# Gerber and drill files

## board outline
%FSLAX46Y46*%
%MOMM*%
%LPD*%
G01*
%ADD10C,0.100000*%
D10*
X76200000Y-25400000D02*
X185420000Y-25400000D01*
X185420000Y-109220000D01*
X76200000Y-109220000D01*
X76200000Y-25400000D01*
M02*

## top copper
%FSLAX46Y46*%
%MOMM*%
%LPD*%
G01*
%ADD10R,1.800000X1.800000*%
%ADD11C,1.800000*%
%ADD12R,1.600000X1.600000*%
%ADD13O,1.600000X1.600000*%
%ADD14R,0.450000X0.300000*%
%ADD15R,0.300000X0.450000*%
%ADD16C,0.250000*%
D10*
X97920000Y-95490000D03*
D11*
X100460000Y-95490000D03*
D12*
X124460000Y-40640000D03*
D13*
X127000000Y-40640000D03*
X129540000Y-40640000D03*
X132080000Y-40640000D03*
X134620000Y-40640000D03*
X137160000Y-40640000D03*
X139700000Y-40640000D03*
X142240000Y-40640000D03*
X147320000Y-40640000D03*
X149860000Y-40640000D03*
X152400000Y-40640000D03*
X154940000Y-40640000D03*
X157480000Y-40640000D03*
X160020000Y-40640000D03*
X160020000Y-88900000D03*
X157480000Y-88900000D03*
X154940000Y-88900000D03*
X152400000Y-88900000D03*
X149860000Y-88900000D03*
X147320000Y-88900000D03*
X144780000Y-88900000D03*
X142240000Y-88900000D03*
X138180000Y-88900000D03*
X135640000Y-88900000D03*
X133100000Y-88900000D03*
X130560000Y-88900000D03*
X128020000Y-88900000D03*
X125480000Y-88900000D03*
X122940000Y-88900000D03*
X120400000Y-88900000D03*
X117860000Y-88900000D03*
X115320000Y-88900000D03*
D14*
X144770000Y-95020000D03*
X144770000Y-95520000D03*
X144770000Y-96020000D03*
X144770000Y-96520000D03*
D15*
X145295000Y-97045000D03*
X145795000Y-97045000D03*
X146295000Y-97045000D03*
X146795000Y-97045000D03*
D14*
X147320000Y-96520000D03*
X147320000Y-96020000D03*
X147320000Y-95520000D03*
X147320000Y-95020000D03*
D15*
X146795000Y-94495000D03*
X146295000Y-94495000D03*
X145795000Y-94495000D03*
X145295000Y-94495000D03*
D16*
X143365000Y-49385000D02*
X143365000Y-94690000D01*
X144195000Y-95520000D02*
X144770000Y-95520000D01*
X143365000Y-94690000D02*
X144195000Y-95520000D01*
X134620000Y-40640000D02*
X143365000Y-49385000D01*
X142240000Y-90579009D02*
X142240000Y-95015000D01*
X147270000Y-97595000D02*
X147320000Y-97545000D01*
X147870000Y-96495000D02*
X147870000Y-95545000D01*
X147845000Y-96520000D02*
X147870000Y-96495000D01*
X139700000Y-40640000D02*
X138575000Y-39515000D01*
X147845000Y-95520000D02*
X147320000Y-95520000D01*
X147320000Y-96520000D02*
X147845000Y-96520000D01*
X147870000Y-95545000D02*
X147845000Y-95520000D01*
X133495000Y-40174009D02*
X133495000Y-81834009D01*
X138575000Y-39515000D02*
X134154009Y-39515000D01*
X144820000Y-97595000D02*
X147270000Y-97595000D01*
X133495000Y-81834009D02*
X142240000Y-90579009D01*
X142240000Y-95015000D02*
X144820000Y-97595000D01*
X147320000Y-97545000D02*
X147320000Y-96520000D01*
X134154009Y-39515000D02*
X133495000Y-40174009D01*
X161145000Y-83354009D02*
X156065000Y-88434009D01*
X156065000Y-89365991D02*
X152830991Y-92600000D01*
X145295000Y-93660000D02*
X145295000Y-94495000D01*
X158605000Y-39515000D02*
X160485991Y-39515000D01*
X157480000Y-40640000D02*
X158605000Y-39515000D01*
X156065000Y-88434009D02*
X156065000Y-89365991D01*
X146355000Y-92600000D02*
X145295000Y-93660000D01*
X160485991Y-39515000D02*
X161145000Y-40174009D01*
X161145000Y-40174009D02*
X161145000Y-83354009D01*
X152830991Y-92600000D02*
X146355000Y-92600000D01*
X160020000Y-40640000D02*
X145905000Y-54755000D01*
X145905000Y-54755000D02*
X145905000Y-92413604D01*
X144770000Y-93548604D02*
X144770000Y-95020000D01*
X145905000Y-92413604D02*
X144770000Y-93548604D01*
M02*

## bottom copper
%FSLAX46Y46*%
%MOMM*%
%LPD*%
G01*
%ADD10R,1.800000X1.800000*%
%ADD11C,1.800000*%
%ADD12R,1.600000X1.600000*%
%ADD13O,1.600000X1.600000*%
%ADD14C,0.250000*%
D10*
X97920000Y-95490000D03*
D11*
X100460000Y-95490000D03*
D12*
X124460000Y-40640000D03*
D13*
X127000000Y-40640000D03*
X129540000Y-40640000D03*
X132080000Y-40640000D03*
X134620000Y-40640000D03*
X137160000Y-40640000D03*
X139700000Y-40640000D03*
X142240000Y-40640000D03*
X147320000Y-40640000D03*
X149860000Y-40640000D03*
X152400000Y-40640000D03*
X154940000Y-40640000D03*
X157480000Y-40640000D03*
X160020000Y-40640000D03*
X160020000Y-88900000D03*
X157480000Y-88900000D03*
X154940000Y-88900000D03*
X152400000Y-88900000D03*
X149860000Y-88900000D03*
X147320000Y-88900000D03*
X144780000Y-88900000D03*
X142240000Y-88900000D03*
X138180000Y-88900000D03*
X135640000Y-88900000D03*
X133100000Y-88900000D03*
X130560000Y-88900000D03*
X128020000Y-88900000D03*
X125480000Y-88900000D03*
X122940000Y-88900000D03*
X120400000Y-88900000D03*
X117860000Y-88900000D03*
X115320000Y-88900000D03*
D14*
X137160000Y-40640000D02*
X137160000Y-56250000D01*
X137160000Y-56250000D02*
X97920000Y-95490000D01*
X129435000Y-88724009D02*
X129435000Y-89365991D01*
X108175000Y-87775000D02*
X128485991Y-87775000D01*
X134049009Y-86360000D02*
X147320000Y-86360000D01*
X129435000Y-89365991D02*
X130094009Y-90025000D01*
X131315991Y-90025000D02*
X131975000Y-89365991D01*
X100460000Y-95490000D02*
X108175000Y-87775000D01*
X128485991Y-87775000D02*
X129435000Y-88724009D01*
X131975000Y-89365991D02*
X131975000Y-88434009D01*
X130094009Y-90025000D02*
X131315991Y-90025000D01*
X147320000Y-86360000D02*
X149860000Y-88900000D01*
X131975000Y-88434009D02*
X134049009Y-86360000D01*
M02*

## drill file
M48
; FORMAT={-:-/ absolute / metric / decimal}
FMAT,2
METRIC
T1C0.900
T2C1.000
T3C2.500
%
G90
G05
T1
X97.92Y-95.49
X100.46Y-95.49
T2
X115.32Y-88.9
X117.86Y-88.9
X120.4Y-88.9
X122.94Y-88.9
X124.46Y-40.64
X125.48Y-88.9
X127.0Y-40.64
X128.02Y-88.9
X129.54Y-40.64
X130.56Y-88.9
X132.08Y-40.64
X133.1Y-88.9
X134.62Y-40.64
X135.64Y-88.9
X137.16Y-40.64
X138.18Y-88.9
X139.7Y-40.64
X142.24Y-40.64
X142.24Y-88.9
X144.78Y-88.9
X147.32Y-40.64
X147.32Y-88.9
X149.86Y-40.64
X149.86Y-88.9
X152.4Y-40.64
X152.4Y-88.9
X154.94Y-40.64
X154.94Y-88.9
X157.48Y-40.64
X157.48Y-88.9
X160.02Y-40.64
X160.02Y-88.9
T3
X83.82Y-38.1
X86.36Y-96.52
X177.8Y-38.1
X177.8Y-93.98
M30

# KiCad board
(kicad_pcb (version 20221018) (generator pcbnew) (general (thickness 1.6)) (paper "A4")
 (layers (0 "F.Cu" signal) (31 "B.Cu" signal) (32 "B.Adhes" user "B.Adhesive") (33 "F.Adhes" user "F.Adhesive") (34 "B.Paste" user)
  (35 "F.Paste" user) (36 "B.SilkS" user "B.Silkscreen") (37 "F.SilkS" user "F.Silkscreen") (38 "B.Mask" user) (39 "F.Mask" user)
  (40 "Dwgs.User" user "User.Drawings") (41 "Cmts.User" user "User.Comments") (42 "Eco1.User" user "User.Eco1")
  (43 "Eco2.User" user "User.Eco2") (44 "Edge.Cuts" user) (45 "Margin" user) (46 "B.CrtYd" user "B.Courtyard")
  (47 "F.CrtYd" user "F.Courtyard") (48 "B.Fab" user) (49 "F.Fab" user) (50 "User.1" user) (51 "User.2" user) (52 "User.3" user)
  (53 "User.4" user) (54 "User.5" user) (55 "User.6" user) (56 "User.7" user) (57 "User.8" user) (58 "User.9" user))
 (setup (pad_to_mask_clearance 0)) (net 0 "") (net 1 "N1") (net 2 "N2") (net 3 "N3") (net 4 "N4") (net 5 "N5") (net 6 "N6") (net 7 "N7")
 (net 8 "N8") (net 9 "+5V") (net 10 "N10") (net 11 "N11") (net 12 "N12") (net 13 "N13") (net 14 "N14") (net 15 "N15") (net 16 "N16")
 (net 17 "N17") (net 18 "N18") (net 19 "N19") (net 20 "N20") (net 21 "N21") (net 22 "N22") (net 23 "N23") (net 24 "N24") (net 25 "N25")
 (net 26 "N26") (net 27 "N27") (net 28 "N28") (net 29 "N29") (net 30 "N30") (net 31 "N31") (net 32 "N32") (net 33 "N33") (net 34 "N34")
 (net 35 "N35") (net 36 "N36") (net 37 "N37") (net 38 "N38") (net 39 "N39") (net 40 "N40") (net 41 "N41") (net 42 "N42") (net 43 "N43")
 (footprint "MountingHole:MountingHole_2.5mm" (layer "F.Cu") (at 83.82 38.1)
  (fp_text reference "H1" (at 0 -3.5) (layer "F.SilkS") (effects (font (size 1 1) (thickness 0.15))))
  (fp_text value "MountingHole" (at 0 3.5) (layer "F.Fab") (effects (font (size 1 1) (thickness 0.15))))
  (pad "" np_thru_hole circle (at 0 0) (size 2.5 2.5) (drill 2.5) (layers "*.Cu" "*.Mask")))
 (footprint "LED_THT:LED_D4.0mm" (layer "F.Cu") (at 97.92 95.49)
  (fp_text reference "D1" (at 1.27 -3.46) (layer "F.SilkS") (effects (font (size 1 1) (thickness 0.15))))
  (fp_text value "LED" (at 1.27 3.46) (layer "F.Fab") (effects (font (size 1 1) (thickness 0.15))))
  (pad "1" thru_hole rect (at 0 0) (size 1.8 1.8) (drill 0.9) (layers "*.Cu" "*.Mask") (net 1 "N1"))
  (pad "2" thru_hole circle (at 2.54 0) (size 1.8 1.8) (drill 0.9) (layers "*.Cu" "*.Mask") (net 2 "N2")))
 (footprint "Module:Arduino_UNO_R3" (layer "F.Cu") (at 124.46 40.64)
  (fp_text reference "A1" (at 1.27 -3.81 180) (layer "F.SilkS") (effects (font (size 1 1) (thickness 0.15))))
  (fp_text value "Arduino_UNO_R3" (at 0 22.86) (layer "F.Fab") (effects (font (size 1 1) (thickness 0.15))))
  (pad "1" thru_hole rect (at 0 0 90) (size 1.6 1.6) (drill 1) (layers "*.Cu" "*.Mask") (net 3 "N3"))
  (pad "2" thru_hole oval (at 2.54 0 90) (size 1.6 1.6) (drill 1) (layers "*.Cu" "*.Mask") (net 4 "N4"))
  (pad "3" thru_hole oval (at 5.08 0 90) (size 1.6 1.6) (drill 1) (layers "*.Cu" "*.Mask") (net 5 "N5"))
  (pad "4" thru_hole oval (at 7.62 0 90) (size 1.6 1.6) (drill 1) (layers "*.Cu" "*.Mask") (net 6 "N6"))
  (pad "5" thru_hole oval (at 10.16 0 90) (size 1.6 1.6) (drill 1) (layers "*.Cu" "*.Mask") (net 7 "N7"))
  (pad "6" thru_hole oval (at 12.7 0 90) (size 1.6 1.6) (drill 1) (layers "*.Cu" "*.Mask") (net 1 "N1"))
  (pad "7" thru_hole oval (at 15.24 0 90) (size 1.6 1.6) (drill 1) (layers "*.Cu" "*.Mask") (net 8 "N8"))
  (pad "8" thru_hole oval (at 17.78 0 90) (size 1.6 1.6) (drill 1) (layers "*.Cu" "*.Mask") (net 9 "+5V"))
  (pad "9" thru_hole oval (at 22.86 0 90) (size 1.6 1.6) (drill 1) (layers "*.Cu" "*.Mask") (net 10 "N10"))
  (pad "10" thru_hole oval (at 25.4 0 90) (size 1.6 1.6) (drill 1) (layers "*.Cu" "*.Mask") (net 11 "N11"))
  (pad "11" thru_hole oval (at 27.94 0 90) (size 1.6 1.6) (drill 1) (layers "*.Cu" "*.Mask") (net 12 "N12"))
  (pad "12" thru_hole oval (at 30.48 0 90) (size 1.6 1.6) (drill 1) (layers "*.Cu" "*.Mask") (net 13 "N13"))
  (pad "13" thru_hole oval (at 33.02 0 90) (size 1.6 1.6) (drill 1) (layers "*.Cu" "*.Mask") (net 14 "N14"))
  (pad "14" thru_hole oval (at 35.56 0 90) (size 1.6 1.6) (drill 1) (layers "*.Cu" "*.Mask") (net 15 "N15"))
  (pad "15" thru_hole oval (at 35.56 48.26 90) (size 1.6 1.6) (drill 1) (layers "*.Cu" "*.Mask") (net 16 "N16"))
  (pad "16" thru_hole oval (at 33.02 48.26 90) (size 1.6 1.6) (drill 1) (layers "*.Cu" "*.Mask") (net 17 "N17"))
  (pad "17" thru_hole oval (at 30.48 48.26 90) (size 1.6 1.6) (drill 1) (layers "*.Cu" "*.Mask") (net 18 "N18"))
  (pad "18" thru_hole oval (at 27.94 48.26 90) (size 1.6 1.6) (drill 1) (layers "*.Cu" "*.Mask") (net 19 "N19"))
  (pad "19" thru_hole oval (at 25.4 48.26 90) (size 1.6 1.6) (drill 1) (layers "*.Cu" "*.Mask") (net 2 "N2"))
  (pad "20" thru_hole oval (at 22.86 48.26 90) (size 1.6 1.6) (drill 1) (layers "*.Cu" "*.Mask") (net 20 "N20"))
  (pad "21" thru_hole oval (at 20.32 48.26 90) (size 1.6 1.6) (drill 1) (layers "*.Cu" "*.Mask") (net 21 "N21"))
  (pad "22" thru_hole oval (at 17.78 48.26 90) (size 1.6 1.6) (drill 1) (layers "*.Cu" "*.Mask") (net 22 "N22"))
  (pad "23" thru_hole oval (at 13.72 48.26 90) (size 1.6 1.6) (drill 1) (layers "*.Cu" "*.Mask") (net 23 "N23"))
  (pad "24" thru_hole oval (at 11.18 48.26 90) (size 1.6 1.6) (drill 1) (layers "*.Cu" "*.Mask") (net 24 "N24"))
  (pad "25" thru_hole oval (at 8.64 48.26 90) (size 1.6 1.6) (drill 1) (layers "*.Cu" "*.Mask") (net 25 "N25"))
  (pad "26" thru_hole oval (at 6.1 48.26 90) (size 1.6 1.6) (drill 1) (layers "*.Cu" "*.Mask") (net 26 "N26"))
  (pad "27" thru_hole oval (at 3.56 48.26 90) (size 1.6 1.6) (drill 1) (layers "*.Cu" "*.Mask") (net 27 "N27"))
  (pad "28" thru_hole oval (at 1.02 48.26 90) (size 1.6 1.6) (drill 1) (layers "*.Cu" "*.Mask") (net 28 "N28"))
  (pad "29" thru_hole oval (at -1.52 48.26 90) (size 1.6 1.6) (drill 1) (layers "*.Cu" "*.Mask") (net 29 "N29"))
  (pad "30" thru_hole oval (at -4.06 48.26 90) (size 1.6 1.6) (drill 1) (layers "*.Cu" "*.Mask") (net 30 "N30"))
  (pad "31" thru_hole oval (at -6.6 48.26 90) (size 1.6 1.6) (drill 1) (layers "*.Cu" "*.Mask") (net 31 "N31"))
  (pad "32" thru_hole oval (at -9.14 48.26 90) (size 1.6 1.6) (drill 1) (layers "*.Cu" "*.Mask") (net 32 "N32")))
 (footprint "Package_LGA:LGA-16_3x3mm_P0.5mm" (layer "F.Cu") (at 146.045 95.77)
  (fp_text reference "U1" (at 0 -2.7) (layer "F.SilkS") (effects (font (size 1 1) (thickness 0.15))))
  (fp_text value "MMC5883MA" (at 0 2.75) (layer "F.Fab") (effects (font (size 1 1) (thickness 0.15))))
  (pad "1" smd rect (at -1.275 -0.75 90) (size 0.3 0.45) (layers "F.Cu" "F.Paste" "F.Mask") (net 15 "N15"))
  (pad "2" smd rect (at -1.275 -0.25 90) (size 0.3 0.45) (layers "F.Cu" "F.Paste" "F.Mask") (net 7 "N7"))
  (pad "3" smd rect (at -1.275 0.25 90) (size 0.3 0.45) (layers "F.Cu" "F.Paste" "F.Mask") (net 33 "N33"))
  (pad "4" smd rect (at -1.275 0.75 90) (size 0.3 0.45) (layers "F.Cu" "F.Paste" "F.Mask") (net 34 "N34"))
  (pad "5" smd rect (at -0.75 1.275) (size 0.3 0.45) (layers "F.Cu" "F.Paste" "F.Mask") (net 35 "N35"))
  (pad "6" smd rect (at -0.25 1.275) (size 0.3 0.45) (layers "F.Cu" "F.Paste" "F.Mask") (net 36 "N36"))
  (pad "7" smd rect (at 0.25 1.275) (size 0.3 0.45) (layers "F.Cu" "F.Paste" "F.Mask") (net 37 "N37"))
  (pad "8" smd rect (at 0.75 1.275) (size 0.3 0.45) (layers "F.Cu" "F.Paste" "F.Mask") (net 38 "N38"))
  (pad "9" smd rect (at 1.275 0.75 90) (size 0.3 0.45) (layers "F.Cu" "F.Paste" "F.Mask") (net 8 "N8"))
  (pad "10" smd rect (at 1.275 0.25 90) (size 0.3 0.45) (layers "F.Cu" "F.Paste" "F.Mask") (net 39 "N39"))
  (pad "11" smd rect (at 1.275 -0.25 90) (size 0.3 0.45) (layers "F.Cu" "F.Paste" "F.Mask") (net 8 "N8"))
  (pad "12" smd rect (at 1.275 -0.75 90) (size 0.3 0.45) (layers "F.Cu" "F.Paste" "F.Mask") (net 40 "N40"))
  (pad "13" smd rect (at 0.75 -1.275) (size 0.3 0.45) (layers "F.Cu" "F.Paste" "F.Mask") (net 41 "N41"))
  (pad "14" smd rect (at 0.25 -1.275) (size 0.3 0.45) (layers "F.Cu" "F.Paste" "F.Mask") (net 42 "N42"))
  (pad "15" smd rect (at -0.25 -1.275) (size 0.3 0.45) (layers "F.Cu" "F.Paste" "F.Mask") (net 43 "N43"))
  (pad "16" smd rect (at -0.75 -1.275) (size 0.3 0.45) (layers "F.Cu" "F.Paste" "F.Mask") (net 14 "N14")))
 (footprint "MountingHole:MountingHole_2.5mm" (layer "F.Cu") (at 86.36 96.52)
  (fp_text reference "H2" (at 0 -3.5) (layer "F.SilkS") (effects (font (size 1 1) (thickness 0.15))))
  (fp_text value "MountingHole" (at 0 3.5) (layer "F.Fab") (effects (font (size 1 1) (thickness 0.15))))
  (pad "" np_thru_hole circle (at 0 0) (size 2.5 2.5) (drill 2.5) (layers "*.Cu" "*.Mask")))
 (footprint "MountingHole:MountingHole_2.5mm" (layer "F.Cu") (at 177.8 38.1)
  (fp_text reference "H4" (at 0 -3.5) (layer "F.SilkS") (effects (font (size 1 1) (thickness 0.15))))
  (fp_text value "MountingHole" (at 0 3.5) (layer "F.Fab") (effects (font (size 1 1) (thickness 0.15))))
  (pad "" np_thru_hole circle (at 0 0) (size 2.5 2.5) (drill 2.5) (layers "*.Cu" "*.Mask")))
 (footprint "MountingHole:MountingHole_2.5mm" (layer "F.Cu") (at 177.8 93.98)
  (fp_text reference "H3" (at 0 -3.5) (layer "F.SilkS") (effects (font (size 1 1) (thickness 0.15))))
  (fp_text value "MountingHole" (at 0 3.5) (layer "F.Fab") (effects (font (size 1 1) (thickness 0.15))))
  (pad "" np_thru_hole circle (at 0 0) (size 2.5 2.5) (drill 2.5) (layers "*.Cu" "*.Mask")))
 (gr_rect (start 76.2 25.4) (end 185.42 109.22) (stroke (width 0.1) (type default)) (fill none) (layer "Edge.Cuts"))
 (segment (start 143.365 49.385) (end 143.365 94.69) (width 0.25) (layer "F.Cu") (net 7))
 (segment (start 144.195 95.52) (end 144.77 95.52) (width 0.25) (layer "F.Cu") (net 7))
 (segment (start 143.365 94.69) (end 144.195 95.52) (width 0.25) (layer "F.Cu") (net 7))
 (segment (start 134.62 40.64) (end 143.365 49.385) (width 0.25) (layer "F.Cu") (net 7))
 (segment (start 137.16 40.64) (end 137.16 56.25) (width 0.25) (layer "B.Cu") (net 1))
 (segment (start 137.16 56.25) (end 97.92 95.49) (width 0.25) (layer "B.Cu") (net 1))
 (segment (start 142.24 90.579009) (end 142.24 95.015) (width 0.25) (layer "F.Cu") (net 8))
 (segment (start 147.27 97.595) (end 147.32 97.545) (width 0.25) (layer "F.Cu") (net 8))
 (segment (start 147.87 96.495) (end 147.87 95.545) (width 0.25) (layer "F.Cu") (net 8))
 (segment (start 147.845 96.52) (end 147.87 96.495) (width 0.25) (layer "F.Cu") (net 8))
 (segment (start 139.7 40.64) (end 138.575 39.515) (width 0.25) (layer "F.Cu") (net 8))
 (segment (start 147.845 95.52) (end 147.32 95.52) (width 0.25) (layer "F.Cu") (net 8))
 (segment (start 147.32 96.52) (end 147.845 96.52) (width 0.25) (layer "F.Cu") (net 8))
 (segment (start 147.87 95.545) (end 147.845 95.52) (width 0.25) (layer "F.Cu") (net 8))
 (segment (start 133.495 40.174009) (end 133.495 81.834009) (width 0.25) (layer "F.Cu") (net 8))
 (segment (start 138.575 39.515) (end 134.154009 39.515) (width 0.25) (layer "F.Cu") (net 8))
 (segment (start 144.82 97.595) (end 147.27 97.595) (width 0.25) (layer "F.Cu") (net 8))
 (segment (start 133.495 81.834009) (end 142.24 90.579009) (width 0.25) (layer "F.Cu") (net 8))
 (segment (start 142.24 95.015) (end 144.82 97.595) (width 0.25) (layer "F.Cu") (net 8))
 (segment (start 147.32 97.545) (end 147.32 96.52) (width 0.25) (layer "F.Cu") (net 8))
 (segment (start 134.154009 39.515) (end 133.495 40.174009) (width 0.25) (layer "F.Cu") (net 8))
 (segment (start 161.145 83.354009) (end 156.065 88.434009) (width 0.25) (layer "F.Cu") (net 14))
 (segment (start 156.065 89.365991) (end 152.830991 92.6) (width 0.25) (layer "F.Cu") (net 14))
 (segment (start 145.295 93.66) (end 145.295 94.495) (width 0.25) (layer "F.Cu") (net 14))
 (segment (start 158.605 39.515) (end 160.485991 39.515) (width 0.25) (layer "F.Cu") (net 14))
 (segment (start 157.48 40.64) (end 158.605 39.515) (width 0.25) (layer "F.Cu") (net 14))
 (segment (start 156.065 88.434009) (end 156.065 89.365991) (width 0.25) (layer "F.Cu") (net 14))
 (segment (start 146.355 92.6) (end 145.295 93.66) (width 0.25) (layer "F.Cu") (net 14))
 (segment (start 160.485991 39.515) (end 161.145 40.174009) (width 0.25) (layer "F.Cu") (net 14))
 (segment (start 161.145 40.174009) (end 161.145 83.354009) (width 0.25) (layer "F.Cu") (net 14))
 (segment (start 152.830991 92.6) (end 146.355 92.6) (width 0.25) (layer "F.Cu") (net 14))
 (segment (start 160.02 40.64) (end 145.905 54.755) (width 0.25) (layer "F.Cu") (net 15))
 (segment (start 145.905 54.755) (end 145.905 92.413604) (width 0.25) (layer "F.Cu") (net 15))
 (segment (start 144.77 93.548604) (end 144.77 95.02) (width 0.25) (layer "F.Cu") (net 15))
 (segment (start 145.905 92.413604) (end 144.77 93.548604) (width 0.25) (layer "F.Cu") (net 15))
 (segment (start 129.435 88.724009) (end 129.435 89.365991) (width 0.25) (layer "B.Cu") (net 2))
 (segment (start 108.175 87.775) (end 128.485991 87.775) (width 0.25) (layer "B.Cu") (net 2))
 (segment (start 134.049009 86.36) (end 147.32 86.36) (width 0.25) (layer "B.Cu") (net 2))
 (segment (start 129.435 89.365991) (end 130.094009 90.025) (width 0.25) (layer "B.Cu") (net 2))
 (segment (start 131.315991 90.025) (end 131.975 89.365991) (width 0.25) (layer "B.Cu") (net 2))
 (segment (start 100.46 95.49) (end 108.175 87.775) (width 0.25) (layer "B.Cu") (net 2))
 (segment (start 128.485991 87.775) (end 129.435 88.724009) (width 0.25) (layer "B.Cu") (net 2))
 (segment (start 131.975 89.365991) (end 131.975 88.434009) (width 0.25) (layer "B.Cu") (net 2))
 (segment (start 130.094009 90.025) (end 131.315991 90.025) (width 0.25) (layer "B.Cu") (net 2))
 (segment (start 147.32 86.36) (end 149.86 88.9) (width 0.25) (layer "B.Cu") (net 2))
 (segment (start 131.975 88.434009) (end 134.049009 86.36) (width 0.25) (layer "B.Cu") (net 2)))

